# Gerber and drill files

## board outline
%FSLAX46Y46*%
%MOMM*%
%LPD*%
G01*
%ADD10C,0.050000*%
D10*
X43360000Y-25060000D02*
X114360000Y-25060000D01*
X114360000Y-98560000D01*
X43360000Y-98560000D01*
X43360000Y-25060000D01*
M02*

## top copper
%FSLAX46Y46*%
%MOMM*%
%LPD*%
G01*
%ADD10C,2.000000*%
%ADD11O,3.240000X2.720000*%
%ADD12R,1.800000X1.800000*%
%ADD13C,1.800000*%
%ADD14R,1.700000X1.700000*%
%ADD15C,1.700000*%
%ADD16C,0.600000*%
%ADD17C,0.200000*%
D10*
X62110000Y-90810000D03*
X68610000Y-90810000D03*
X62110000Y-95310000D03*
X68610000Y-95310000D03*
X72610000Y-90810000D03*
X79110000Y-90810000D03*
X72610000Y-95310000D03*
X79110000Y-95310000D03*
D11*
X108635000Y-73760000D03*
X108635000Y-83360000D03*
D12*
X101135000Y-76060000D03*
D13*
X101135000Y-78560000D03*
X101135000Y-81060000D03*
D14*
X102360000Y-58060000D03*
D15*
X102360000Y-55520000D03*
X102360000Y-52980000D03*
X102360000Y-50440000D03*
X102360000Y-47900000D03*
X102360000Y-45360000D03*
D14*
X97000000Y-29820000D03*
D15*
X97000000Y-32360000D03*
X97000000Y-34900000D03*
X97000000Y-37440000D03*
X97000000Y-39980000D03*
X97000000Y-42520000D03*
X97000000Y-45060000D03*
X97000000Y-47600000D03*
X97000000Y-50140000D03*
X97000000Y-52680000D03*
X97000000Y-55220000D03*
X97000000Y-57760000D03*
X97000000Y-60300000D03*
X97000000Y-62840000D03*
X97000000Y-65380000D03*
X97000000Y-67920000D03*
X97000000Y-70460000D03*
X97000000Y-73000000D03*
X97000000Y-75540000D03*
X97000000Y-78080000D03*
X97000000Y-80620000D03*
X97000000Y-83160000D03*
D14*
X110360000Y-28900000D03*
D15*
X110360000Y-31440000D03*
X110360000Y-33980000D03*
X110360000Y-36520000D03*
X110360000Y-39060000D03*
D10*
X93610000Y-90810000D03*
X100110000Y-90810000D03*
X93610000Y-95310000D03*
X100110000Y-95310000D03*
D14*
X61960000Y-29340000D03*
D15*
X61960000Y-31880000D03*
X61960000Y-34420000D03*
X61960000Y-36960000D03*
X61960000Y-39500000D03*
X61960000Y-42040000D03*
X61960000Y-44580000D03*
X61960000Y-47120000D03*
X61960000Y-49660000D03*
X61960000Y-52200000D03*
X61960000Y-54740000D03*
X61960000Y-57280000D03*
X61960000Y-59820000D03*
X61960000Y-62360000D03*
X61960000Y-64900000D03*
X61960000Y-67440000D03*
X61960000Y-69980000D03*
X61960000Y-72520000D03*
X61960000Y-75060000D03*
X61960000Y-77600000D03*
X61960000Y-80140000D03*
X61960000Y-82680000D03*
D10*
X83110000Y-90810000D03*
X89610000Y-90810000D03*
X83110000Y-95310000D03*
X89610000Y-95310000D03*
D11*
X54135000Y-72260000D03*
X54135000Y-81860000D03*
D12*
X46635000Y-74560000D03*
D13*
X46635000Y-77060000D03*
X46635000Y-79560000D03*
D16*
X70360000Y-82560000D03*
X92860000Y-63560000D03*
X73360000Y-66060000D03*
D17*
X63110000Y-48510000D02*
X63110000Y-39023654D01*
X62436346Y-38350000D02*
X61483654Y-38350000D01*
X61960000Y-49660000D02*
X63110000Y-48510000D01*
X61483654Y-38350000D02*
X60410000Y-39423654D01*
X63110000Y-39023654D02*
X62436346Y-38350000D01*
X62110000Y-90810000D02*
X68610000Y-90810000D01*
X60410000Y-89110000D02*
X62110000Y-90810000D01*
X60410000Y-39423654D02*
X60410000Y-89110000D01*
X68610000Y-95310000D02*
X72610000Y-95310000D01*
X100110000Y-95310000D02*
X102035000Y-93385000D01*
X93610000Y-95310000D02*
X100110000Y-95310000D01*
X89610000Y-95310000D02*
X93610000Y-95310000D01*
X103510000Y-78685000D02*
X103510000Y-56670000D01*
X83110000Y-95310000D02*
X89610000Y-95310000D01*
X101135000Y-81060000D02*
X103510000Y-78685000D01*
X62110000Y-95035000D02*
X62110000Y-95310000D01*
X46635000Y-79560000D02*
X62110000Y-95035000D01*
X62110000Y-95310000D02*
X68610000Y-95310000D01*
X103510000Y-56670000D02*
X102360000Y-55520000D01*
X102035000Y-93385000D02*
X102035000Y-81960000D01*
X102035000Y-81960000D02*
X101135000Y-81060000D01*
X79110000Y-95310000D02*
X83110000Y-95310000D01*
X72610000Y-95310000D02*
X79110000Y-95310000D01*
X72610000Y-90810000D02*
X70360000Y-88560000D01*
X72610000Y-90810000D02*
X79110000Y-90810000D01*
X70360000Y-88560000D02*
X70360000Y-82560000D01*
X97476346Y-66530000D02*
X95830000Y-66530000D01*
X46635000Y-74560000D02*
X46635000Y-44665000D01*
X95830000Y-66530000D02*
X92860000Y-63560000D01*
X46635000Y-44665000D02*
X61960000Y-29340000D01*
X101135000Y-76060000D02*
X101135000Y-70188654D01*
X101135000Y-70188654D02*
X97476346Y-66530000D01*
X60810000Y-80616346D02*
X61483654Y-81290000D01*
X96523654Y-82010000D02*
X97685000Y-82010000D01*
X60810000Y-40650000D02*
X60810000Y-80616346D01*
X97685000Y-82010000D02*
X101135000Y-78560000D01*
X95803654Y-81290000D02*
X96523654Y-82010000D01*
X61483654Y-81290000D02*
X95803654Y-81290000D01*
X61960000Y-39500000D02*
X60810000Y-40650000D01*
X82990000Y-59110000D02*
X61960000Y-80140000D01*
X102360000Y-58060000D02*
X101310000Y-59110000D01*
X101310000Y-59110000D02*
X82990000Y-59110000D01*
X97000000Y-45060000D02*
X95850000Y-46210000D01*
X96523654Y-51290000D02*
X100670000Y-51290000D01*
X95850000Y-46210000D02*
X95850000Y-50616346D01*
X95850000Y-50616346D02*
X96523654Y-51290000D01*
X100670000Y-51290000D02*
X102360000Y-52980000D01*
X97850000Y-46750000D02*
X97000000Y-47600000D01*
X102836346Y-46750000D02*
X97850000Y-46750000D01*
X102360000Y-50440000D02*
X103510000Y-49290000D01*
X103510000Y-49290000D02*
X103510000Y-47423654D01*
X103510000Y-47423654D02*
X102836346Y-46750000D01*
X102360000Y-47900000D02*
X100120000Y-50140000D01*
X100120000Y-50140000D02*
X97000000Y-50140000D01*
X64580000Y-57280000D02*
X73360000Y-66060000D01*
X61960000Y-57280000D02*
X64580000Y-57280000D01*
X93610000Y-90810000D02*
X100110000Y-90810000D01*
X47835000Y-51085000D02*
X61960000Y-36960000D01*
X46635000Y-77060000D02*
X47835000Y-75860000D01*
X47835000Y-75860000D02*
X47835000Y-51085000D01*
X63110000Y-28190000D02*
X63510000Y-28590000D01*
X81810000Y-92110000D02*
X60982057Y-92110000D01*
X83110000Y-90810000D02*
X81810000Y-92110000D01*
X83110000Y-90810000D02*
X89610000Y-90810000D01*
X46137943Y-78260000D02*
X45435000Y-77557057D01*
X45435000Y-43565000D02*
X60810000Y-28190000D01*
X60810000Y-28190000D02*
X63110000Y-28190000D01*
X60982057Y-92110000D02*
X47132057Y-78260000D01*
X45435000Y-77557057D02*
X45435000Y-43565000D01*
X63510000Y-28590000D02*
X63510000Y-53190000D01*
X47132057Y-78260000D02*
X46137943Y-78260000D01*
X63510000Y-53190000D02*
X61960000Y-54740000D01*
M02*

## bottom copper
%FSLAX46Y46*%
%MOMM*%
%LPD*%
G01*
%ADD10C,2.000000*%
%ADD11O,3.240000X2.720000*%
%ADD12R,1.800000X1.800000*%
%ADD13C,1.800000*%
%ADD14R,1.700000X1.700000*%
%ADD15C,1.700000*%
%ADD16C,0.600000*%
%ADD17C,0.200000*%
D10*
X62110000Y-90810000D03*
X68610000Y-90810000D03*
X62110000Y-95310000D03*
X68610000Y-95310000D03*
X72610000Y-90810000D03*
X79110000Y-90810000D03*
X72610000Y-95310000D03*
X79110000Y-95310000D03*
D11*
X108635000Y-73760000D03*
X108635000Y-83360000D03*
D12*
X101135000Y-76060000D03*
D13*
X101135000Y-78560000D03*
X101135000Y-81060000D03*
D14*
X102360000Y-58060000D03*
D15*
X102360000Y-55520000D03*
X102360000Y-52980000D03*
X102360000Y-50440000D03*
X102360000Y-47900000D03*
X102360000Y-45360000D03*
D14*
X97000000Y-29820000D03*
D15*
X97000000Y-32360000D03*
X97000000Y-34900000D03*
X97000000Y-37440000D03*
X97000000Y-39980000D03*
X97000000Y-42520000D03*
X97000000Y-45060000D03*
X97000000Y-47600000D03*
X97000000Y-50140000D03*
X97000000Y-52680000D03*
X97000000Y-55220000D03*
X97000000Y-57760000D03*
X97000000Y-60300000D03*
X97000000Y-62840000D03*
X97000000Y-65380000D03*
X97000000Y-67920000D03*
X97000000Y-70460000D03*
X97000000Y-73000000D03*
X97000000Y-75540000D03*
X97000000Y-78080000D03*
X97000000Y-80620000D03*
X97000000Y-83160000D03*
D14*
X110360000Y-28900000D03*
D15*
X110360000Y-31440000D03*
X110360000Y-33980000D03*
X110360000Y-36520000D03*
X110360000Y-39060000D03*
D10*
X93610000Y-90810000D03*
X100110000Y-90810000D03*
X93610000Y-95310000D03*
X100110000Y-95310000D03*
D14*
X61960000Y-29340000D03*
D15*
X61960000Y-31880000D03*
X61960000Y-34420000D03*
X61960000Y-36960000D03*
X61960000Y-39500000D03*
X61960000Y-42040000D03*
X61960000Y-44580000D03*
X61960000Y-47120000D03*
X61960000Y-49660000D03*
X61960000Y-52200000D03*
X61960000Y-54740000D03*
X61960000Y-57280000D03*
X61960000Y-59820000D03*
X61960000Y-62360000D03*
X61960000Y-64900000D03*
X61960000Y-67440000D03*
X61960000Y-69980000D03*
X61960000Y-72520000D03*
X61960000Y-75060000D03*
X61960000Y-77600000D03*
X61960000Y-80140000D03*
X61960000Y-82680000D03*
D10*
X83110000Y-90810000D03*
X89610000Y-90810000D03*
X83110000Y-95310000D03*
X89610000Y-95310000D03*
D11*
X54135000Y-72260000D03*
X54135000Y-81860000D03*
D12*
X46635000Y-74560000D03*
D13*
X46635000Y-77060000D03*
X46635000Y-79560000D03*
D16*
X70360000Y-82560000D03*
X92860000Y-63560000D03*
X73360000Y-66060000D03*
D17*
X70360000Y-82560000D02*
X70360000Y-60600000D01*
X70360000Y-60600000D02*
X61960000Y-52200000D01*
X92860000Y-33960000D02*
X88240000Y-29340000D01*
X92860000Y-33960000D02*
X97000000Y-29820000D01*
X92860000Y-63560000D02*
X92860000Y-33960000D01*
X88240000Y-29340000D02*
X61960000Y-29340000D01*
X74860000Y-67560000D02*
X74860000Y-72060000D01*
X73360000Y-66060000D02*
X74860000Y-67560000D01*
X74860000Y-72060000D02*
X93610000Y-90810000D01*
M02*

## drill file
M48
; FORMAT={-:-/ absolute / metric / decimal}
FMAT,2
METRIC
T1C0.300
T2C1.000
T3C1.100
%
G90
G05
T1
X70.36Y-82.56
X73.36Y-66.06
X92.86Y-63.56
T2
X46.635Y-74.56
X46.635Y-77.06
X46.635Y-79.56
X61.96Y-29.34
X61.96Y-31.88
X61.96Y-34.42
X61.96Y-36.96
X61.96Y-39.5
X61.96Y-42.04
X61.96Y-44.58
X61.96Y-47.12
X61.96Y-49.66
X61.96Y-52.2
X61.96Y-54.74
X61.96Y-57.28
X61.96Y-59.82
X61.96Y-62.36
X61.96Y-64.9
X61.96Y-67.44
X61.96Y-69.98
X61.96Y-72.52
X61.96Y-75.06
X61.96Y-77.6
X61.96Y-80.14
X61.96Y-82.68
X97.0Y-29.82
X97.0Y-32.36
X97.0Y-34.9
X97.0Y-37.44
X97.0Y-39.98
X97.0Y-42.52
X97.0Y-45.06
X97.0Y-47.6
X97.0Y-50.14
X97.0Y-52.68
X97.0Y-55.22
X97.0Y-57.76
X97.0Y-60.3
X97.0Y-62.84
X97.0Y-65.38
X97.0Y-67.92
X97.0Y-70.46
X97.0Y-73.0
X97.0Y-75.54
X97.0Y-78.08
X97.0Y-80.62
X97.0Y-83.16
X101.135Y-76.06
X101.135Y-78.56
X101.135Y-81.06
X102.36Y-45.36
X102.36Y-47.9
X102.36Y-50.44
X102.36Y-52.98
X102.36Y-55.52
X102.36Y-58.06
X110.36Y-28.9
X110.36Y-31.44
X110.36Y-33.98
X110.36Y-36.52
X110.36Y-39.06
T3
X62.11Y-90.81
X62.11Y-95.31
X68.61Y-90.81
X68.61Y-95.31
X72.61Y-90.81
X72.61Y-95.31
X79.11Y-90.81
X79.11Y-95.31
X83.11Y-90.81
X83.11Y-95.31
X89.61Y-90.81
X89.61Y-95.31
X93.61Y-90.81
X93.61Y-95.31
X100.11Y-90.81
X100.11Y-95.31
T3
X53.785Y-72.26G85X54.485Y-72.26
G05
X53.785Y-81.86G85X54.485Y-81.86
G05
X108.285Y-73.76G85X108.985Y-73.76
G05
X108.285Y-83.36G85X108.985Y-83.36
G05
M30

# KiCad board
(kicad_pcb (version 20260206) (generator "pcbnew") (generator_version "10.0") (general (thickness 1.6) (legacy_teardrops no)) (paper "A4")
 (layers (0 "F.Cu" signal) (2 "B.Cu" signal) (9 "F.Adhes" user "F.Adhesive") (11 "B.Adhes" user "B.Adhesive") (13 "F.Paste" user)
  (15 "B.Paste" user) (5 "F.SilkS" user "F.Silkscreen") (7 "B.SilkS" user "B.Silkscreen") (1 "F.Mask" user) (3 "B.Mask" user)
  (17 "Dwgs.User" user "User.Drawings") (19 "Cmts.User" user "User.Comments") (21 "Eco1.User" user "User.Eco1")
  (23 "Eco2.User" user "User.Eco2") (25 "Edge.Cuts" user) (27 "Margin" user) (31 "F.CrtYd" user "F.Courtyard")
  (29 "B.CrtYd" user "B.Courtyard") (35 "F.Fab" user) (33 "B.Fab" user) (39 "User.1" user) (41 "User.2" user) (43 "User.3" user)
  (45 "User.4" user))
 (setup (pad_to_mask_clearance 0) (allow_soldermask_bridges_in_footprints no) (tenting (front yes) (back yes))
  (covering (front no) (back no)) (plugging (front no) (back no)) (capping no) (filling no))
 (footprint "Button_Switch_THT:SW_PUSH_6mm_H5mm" (layer "F.Cu") (at 62.11 90.81)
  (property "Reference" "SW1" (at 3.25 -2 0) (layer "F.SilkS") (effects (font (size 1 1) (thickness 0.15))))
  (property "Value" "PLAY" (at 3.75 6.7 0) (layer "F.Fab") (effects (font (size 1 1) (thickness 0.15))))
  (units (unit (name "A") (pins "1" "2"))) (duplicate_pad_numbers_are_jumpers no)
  (pad "1" thru_hole circle (at 0 0 90) (size 2 2) (drill 1.1) (layers "*.Cu" "*.Mask") (remove_unused_layers no) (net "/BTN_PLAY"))
  (pad "1" thru_hole circle (at 6.5 0 90) (size 2 2) (drill 1.1) (layers "*.Cu" "*.Mask") (remove_unused_layers no) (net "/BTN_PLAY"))
  (pad "2" thru_hole circle (at 0 4.5 90) (size 2 2) (drill 1.1) (layers "*.Cu" "*.Mask") (remove_unused_layers no) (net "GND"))
  (pad "2" thru_hole circle (at 6.5 4.5 90) (size 2 2) (drill 1.1) (layers "*.Cu" "*.Mask") (remove_unused_layers no) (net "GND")))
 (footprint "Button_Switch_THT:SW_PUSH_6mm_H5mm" (layer "F.Cu") (at 72.61 90.81)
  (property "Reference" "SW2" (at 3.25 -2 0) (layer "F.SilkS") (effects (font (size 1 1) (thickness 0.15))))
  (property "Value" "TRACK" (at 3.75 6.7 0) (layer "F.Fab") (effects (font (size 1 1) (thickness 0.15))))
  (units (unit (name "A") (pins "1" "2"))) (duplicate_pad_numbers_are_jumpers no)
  (pad "1" thru_hole circle (at 0 0 90) (size 2 2) (drill 1.1) (layers "*.Cu" "*.Mask") (remove_unused_layers no) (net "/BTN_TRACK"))
  (pad "1" thru_hole circle (at 6.5 0 90) (size 2 2) (drill 1.1) (layers "*.Cu" "*.Mask") (remove_unused_layers no) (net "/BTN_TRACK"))
  (pad "2" thru_hole circle (at 0 4.5 90) (size 2 2) (drill 1.1) (layers "*.Cu" "*.Mask") (remove_unused_layers no) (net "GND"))
  (pad "2" thru_hole circle (at 6.5 4.5 90) (size 2 2) (drill 1.1) (layers "*.Cu" "*.Mask") (remove_unused_layers no) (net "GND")))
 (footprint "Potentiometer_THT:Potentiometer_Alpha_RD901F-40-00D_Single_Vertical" (layer "F.Cu") (at 101.135 76.06)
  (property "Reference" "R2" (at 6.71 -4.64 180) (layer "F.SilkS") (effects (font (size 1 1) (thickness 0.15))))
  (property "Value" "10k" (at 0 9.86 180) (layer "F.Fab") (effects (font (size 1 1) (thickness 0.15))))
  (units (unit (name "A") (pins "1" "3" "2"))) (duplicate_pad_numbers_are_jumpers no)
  (pad "" thru_hole oval (at 7.5 -2.3 90) (size 2.72 3.24) (drill oval 1.1 1.8) (layers "*.Cu" "*.Mask") (remove_unused_layers no))
  (pad "" thru_hole oval (at 7.5 7.3 90) (size 2.72 3.24) (drill oval 1.1 1.8) (layers "*.Cu" "*.Mask") (remove_unused_layers no))
  (pad "1" thru_hole rect (at 0 0 90) (size 1.8 1.8) (drill 1) (layers "*.Cu" "*.Mask") (remove_unused_layers no) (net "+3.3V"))
  (pad "2" thru_hole circle (at 0 2.5 90) (size 1.8 1.8) (drill 1) (layers "*.Cu" "*.Mask") (remove_unused_layers no) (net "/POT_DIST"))
  (pad "3" thru_hole circle (at 0 5 90) (size 1.8 1.8) (drill 1) (layers "*.Cu" "*.Mask") (remove_unused_layers no) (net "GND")))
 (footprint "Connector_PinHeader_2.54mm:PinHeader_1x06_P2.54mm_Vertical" (layer "F.Cu") (at 102.36 58.06 180)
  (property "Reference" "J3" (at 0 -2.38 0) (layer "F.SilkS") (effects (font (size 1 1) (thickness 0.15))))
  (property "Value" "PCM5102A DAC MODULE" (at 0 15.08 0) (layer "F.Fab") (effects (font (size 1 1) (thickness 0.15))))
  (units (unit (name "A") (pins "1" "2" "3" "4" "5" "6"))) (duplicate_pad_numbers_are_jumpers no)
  (pad "1" thru_hole rect (at 0 0 180) (size 1.7 1.7) (drill 1) (layers "*.Cu" "*.Mask") (remove_unused_layers no) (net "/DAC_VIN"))
  (pad "2" thru_hole circle (at 0 2.54 180) (size 1.7 1.7) (drill 1) (layers "*.Cu" "*.Mask") (remove_unused_layers no) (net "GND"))
  (pad "3" thru_hole circle (at 0 5.08 180) (size 1.7 1.7) (drill 1) (layers "*.Cu" "*.Mask") (remove_unused_layers no) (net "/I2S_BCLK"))
  (pad "4" thru_hole circle (at 0 7.62 180) (size 1.7 1.7) (drill 1) (layers "*.Cu" "*.Mask") (remove_unused_layers no) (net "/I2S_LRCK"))
  (pad "5" thru_hole circle (at 0 10.16 180) (size 1.7 1.7) (drill 1) (layers "*.Cu" "*.Mask") (remove_unused_layers no) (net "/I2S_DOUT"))
  (pad "6" thru_hole circle (at 0 12.7 180) (size 1.7 1.7) (drill 1) (layers "*.Cu" "*.Mask") (remove_unused_layers no) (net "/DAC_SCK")))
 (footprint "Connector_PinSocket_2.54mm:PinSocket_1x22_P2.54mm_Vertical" (layer "F.Cu") (at 97 29.82)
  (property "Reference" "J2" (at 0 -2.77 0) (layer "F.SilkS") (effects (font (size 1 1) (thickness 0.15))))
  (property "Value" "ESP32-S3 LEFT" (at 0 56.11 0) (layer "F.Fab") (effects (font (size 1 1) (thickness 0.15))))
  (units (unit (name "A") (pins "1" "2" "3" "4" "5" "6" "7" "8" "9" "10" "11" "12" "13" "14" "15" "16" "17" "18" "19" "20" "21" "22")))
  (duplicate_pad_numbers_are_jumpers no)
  (pad "1" thru_hole rect (at 0 0) (size 1.7 1.7) (drill 1) (layers "*.Cu" "*.Mask") (remove_unused_layers no) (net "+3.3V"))
  (pad "2" thru_hole circle (at 0 2.54) (size 1.7 1.7) (drill 1) (layers "*.Cu" "*.Mask") (remove_unused_layers no)
   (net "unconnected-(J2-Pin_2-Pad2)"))
  (pad "3" thru_hole circle (at 0 5.08) (size 1.7 1.7) (drill 1) (layers "*.Cu" "*.Mask") (remove_unused_layers no)
   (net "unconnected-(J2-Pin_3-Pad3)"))
  (pad "4" thru_hole circle (at 0 7.62) (size 1.7 1.7) (drill 1) (layers "*.Cu" "*.Mask") (remove_unused_layers no)
   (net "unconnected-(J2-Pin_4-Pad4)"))
  (pad "5" thru_hole circle (at 0 10.16) (size 1.7 1.7) (drill 1) (layers "*.Cu" "*.Mask") (remove_unused_layers no)
   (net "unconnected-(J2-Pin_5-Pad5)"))
  (pad "6" thru_hole circle (at 0 12.7) (size 1.7 1.7) (drill 1) (layers "*.Cu" "*.Mask") (remove_unused_layers no)
   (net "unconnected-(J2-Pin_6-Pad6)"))
  (pad "7" thru_hole circle (at 0 15.24) (size 1.7 1.7) (drill 1) (layers "*.Cu" "*.Mask") (remove_unused_layers no) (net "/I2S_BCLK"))
  (pad "8" thru_hole circle (at 0 17.78) (size 1.7 1.7) (drill 1) (layers "*.Cu" "*.Mask") (remove_unused_layers no) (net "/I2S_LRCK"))
  (pad "9" thru_hole circle (at 0 20.32) (size 1.7 1.7) (drill 1) (layers "*.Cu" "*.Mask") (remove_unused_layers no) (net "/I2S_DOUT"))
  (pad "10" thru_hole circle (at 0 22.86) (size 1.7 1.7) (drill 1) (layers "*.Cu" "*.Mask") (remove_unused_layers no)
   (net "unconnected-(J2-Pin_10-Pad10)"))
  (pad "11" thru_hole circle (at 0 25.4) (size 1.7 1.7) (drill 1) (layers "*.Cu" "*.Mask") (remove_unused_layers no)
   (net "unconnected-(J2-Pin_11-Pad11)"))
  (pad "12" thru_hole circle (at 0 27.94) (size 1.7 1.7) (drill 1) (layers "*.Cu" "*.Mask") (remove_unused_layers no)
   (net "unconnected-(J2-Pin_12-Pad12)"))
  (pad "13" thru_hole circle (at 0 30.48) (size 1.7 1.7) (drill 1) (layers "*.Cu" "*.Mask") (remove_unused_layers no)
   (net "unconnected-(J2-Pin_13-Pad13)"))
  (pad "14" thru_hole circle (at 0 33.02) (size 1.7 1.7) (drill 1) (layers "*.Cu" "*.Mask") (remove_unused_layers no)
   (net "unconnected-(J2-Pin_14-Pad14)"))
  (pad "15" thru_hole circle (at 0 35.56) (size 1.7 1.7) (drill 1) (layers "*.Cu" "*.Mask") (remove_unused_layers no)
   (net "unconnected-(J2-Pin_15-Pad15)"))
  (pad "16" thru_hole circle (at 0 38.1) (size 1.7 1.7) (drill 1) (layers "*.Cu" "*.Mask") (remove_unused_layers no)
   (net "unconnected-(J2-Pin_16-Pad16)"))
  (pad "17" thru_hole circle (at 0 40.64) (size 1.7 1.7) (drill 1) (layers "*.Cu" "*.Mask") (remove_unused_layers no)
   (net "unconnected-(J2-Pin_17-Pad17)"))
  (pad "18" thru_hole circle (at 0 43.18) (size 1.7 1.7) (drill 1) (layers "*.Cu" "*.Mask") (remove_unused_layers no)
   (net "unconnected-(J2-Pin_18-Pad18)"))
  (pad "19" thru_hole circle (at 0 45.72) (size 1.7 1.7) (drill 1) (layers "*.Cu" "*.Mask") (remove_unused_layers no)
   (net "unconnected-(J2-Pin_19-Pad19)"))
  (pad "20" thru_hole circle (at 0 48.26) (size 1.7 1.7) (drill 1) (layers "*.Cu" "*.Mask") (remove_unused_layers no)
   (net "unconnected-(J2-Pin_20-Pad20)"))
  (pad "21" thru_hole circle (at 0 50.8) (size 1.7 1.7) (drill 1) (layers "*.Cu" "*.Mask") (remove_unused_layers no)
   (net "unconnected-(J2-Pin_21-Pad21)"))
  (pad "22" thru_hole circle (at 0 53.34) (size 1.7 1.7) (drill 1) (layers "*.Cu" "*.Mask") (remove_unused_layers no)
   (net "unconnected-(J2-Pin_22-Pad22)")))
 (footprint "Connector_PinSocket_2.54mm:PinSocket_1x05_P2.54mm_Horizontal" (layer "F.Cu") (at 110.36 28.9)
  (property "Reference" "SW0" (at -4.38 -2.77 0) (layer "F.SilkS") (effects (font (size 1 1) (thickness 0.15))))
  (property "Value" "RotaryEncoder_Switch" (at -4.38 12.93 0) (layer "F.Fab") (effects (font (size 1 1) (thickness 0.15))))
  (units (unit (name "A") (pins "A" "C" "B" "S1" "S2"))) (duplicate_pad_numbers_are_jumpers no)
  (pad "1" thru_hole rect (at 0 0) (size 1.7 1.7) (drill 1) (layers "*.Cu" "*.Mask") (remove_unused_layers no))
  (pad "2" thru_hole circle (at 0 2.54) (size 1.7 1.7) (drill 1) (layers "*.Cu" "*.Mask") (remove_unused_layers no))
  (pad "3" thru_hole circle (at 0 5.08) (size 1.7 1.7) (drill 1) (layers "*.Cu" "*.Mask") (remove_unused_layers no))
  (pad "4" thru_hole circle (at 0 7.62) (size 1.7 1.7) (drill 1) (layers "*.Cu" "*.Mask") (remove_unused_layers no))
  (pad "5" thru_hole circle (at 0 10.16) (size 1.7 1.7) (drill 1) (layers "*.Cu" "*.Mask") (remove_unused_layers no)))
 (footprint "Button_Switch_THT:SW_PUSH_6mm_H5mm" (layer "F.Cu") (at 93.61 90.81)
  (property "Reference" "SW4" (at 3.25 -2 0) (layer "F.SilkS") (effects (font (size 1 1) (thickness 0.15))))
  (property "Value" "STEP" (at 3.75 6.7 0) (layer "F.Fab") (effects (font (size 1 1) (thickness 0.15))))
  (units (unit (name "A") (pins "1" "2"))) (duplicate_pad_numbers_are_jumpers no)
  (pad "1" thru_hole circle (at 0 0 90) (size 2 2) (drill 1.1) (layers "*.Cu" "*.Mask") (remove_unused_layers no) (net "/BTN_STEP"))
  (pad "1" thru_hole circle (at 6.5 0 90) (size 2 2) (drill 1.1) (layers "*.Cu" "*.Mask") (remove_unused_layers no) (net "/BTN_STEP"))
  (pad "2" thru_hole circle (at 0 4.5 90) (size 2 2) (drill 1.1) (layers "*.Cu" "*.Mask") (remove_unused_layers no) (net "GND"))
  (pad "2" thru_hole circle (at 6.5 4.5 90) (size 2 2) (drill 1.1) (layers "*.Cu" "*.Mask") (remove_unused_layers no) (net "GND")))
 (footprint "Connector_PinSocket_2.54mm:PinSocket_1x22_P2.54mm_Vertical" (layer "F.Cu") (at 61.96 29.34)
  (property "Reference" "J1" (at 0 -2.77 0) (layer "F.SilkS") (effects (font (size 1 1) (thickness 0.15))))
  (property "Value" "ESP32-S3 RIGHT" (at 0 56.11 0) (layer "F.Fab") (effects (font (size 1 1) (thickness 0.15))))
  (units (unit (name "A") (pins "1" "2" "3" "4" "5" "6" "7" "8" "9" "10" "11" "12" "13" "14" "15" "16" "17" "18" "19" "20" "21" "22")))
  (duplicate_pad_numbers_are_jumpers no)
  (pad "1" thru_hole rect (at 0 0) (size 1.7 1.7) (drill 1) (layers "*.Cu" "*.Mask") (remove_unused_layers no) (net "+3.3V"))
  (pad "2" thru_hole circle (at 0 2.54) (size 1.7 1.7) (drill 1) (layers "*.Cu" "*.Mask") (remove_unused_layers no)
   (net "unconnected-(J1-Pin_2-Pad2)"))
  (pad "3" thru_hole circle (at 0 5.08) (size 1.7 1.7) (drill 1) (layers "*.Cu" "*.Mask") (remove_unused_layers no)
   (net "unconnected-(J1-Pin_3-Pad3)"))
  (pad "4" thru_hole circle (at 0 7.62) (size 1.7 1.7) (drill 1) (layers "*.Cu" "*.Mask") (remove_unused_layers no) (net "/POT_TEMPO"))
  (pad "5" thru_hole circle (at 0 10.16) (size 1.7 1.7) (drill 1) (layers "*.Cu" "*.Mask") (remove_unused_layers no) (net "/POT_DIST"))
  (pad "6" thru_hole circle (at 0 12.7) (size 1.7 1.7) (drill 1) (layers "*.Cu" "*.Mask") (remove_unused_layers no) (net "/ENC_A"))
  (pad "7" thru_hole circle (at 0 15.24) (size 1.7 1.7) (drill 1) (layers "*.Cu" "*.Mask") (remove_unused_layers no) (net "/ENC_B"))
  (pad "8" thru_hole circle (at 0 17.78) (size 1.7 1.7) (drill 1) (layers "*.Cu" "*.Mask") (remove_unused_layers no) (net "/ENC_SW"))
  (pad "9" thru_hole circle (at 0 20.32) (size 1.7 1.7) (drill 1) (layers "*.Cu" "*.Mask") (remove_unused_layers no) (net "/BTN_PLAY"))
  (pad "10" thru_hole circle (at 0 22.86) (size 1.7 1.7) (drill 1) (layers "*.Cu" "*.Mask") (remove_unused_layers no) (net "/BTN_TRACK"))
  (pad "11" thru_hole circle (at 0 25.4) (size 1.7 1.7) (drill 1) (layers "*.Cu" "*.Mask") (remove_unused_layers no) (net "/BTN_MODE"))
  (pad "12" thru_hole circle (at 0 27.94) (size 1.7 1.7) (drill 1) (layers "*.Cu" "*.Mask") (remove_unused_layers no) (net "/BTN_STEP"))
  (pad "13" thru_hole circle (at 0 30.48) (size 1.7 1.7) (drill 1) (layers "*.Cu" "*.Mask") (remove_unused_layers no)
   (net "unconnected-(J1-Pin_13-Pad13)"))
  (pad "14" thru_hole circle (at 0 33.02) (size 1.7 1.7) (drill 1) (layers "*.Cu" "*.Mask") (remove_unused_layers no)
   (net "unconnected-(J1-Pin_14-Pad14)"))
  (pad "15" thru_hole circle (at 0 35.56) (size 1.7 1.7) (drill 1) (layers "*.Cu" "*.Mask") (remove_unused_layers no)
   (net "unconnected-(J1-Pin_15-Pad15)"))
  (pad "16" thru_hole circle (at 0 38.1) (size 1.7 1.7) (drill 1) (layers "*.Cu" "*.Mask") (remove_unused_layers no)
   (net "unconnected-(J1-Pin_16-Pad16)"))
  (pad "17" thru_hole circle (at 0 40.64) (size 1.7 1.7) (drill 1) (layers "*.Cu" "*.Mask") (remove_unused_layers no)
   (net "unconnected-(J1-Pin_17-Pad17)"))
  (pad "18" thru_hole circle (at 0 43.18) (size 1.7 1.7) (drill 1) (layers "*.Cu" "*.Mask") (remove_unused_layers no)
   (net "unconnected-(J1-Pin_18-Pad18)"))
  (pad "19" thru_hole circle (at 0 45.72) (size 1.7 1.7) (drill 1) (layers "*.Cu" "*.Mask") (remove_unused_layers no)
   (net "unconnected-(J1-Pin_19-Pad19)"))
  (pad "20" thru_hole circle (at 0 48.26) (size 1.7 1.7) (drill 1) (layers "*.Cu" "*.Mask") (remove_unused_layers no)
   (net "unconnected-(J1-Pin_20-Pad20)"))
  (pad "21" thru_hole circle (at 0 50.8) (size 1.7 1.7) (drill 1) (layers "*.Cu" "*.Mask") (remove_unused_layers no) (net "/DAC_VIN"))
  (pad "22" thru_hole circle (at 0 53.34) (size 1.7 1.7) (drill 1) (layers "*.Cu" "*.Mask") (remove_unused_layers no)
   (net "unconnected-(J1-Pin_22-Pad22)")))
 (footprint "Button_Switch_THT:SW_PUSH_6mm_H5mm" (layer "F.Cu") (at 83.11 90.81)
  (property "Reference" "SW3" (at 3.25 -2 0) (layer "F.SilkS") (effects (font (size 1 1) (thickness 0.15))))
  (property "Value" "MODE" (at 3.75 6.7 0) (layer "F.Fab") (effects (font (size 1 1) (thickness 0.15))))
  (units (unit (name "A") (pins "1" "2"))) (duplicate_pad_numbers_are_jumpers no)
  (pad "1" thru_hole circle (at 0 0 90) (size 2 2) (drill 1.1) (layers "*.Cu" "*.Mask") (remove_unused_layers no) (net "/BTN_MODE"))
  (pad "1" thru_hole circle (at 6.5 0 90) (size 2 2) (drill 1.1) (layers "*.Cu" "*.Mask") (remove_unused_layers no) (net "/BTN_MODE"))
  (pad "2" thru_hole circle (at 0 4.5 90) (size 2 2) (drill 1.1) (layers "*.Cu" "*.Mask") (remove_unused_layers no) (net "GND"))
  (pad "2" thru_hole circle (at 6.5 4.5 90) (size 2 2) (drill 1.1) (layers "*.Cu" "*.Mask") (remove_unused_layers no) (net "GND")))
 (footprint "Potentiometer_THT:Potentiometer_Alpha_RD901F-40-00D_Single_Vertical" (layer "F.Cu") (at 46.635 74.56)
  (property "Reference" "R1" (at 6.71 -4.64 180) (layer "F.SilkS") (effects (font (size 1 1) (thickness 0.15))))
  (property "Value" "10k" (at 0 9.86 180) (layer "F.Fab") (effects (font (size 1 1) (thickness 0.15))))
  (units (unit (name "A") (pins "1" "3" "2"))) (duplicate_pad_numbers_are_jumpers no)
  (pad "" thru_hole oval (at 7.5 -2.3 90) (size 2.72 3.24) (drill oval 1.1 1.8) (layers "*.Cu" "*.Mask") (remove_unused_layers no))
  (pad "" thru_hole oval (at 7.5 7.3 90) (size 2.72 3.24) (drill oval 1.1 1.8) (layers "*.Cu" "*.Mask") (remove_unused_layers no))
  (pad "1" thru_hole rect (at 0 0 90) (size 1.8 1.8) (drill 1) (layers "*.Cu" "*.Mask") (remove_unused_layers no) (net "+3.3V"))
  (pad "2" thru_hole circle (at 0 2.5 90) (size 1.8 1.8) (drill 1) (layers "*.Cu" "*.Mask") (remove_unused_layers no) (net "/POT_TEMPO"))
  (pad "3" thru_hole circle (at 0 5 90) (size 1.8 1.8) (drill 1) (layers "*.Cu" "*.Mask") (remove_unused_layers no) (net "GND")))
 (gr_rect (start 43.36 25.06) (end 114.36 98.56) (stroke (width 0.05) (type default)) (fill no) (layer "Edge.Cuts"))
 (segment (start 63.11 48.51) (end 63.11 39.023654) (width 0.2) (layer "F.Cu") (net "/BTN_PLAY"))
 (segment (start 62.436346 38.35) (end 61.483654 38.35) (width 0.2) (layer "F.Cu") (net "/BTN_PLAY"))
 (segment (start 61.96 49.66) (end 63.11 48.51) (width 0.2) (layer "F.Cu") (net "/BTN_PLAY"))
 (segment (start 61.483654 38.35) (end 60.41 39.423654) (width 0.2) (layer "F.Cu") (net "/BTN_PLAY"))
 (segment (start 63.11 39.023654) (end 62.436346 38.35) (width 0.2) (layer "F.Cu") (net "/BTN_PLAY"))
 (segment (start 62.11 90.81) (end 68.61 90.81) (width 0.2) (layer "F.Cu") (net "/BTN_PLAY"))
 (segment (start 60.41 89.11) (end 62.11 90.81) (width 0.2) (layer "F.Cu") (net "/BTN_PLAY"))
 (segment (start 60.41 39.423654) (end 60.41 89.11) (width 0.2) (layer "F.Cu") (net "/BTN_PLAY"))
 (segment (start 68.61 95.31) (end 72.61 95.31) (width 0.2) (layer "F.Cu") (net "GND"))
 (segment (start 100.11 95.31) (end 102.035 93.385) (width 0.2) (layer "F.Cu") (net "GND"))
 (segment (start 93.61 95.31) (end 100.11 95.31) (width 0.2) (layer "F.Cu") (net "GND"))
 (segment (start 89.61 95.31) (end 93.61 95.31) (width 0.2) (layer "F.Cu") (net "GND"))
 (segment (start 103.51 78.685) (end 103.51 56.67) (width 0.2) (layer "F.Cu") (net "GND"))
 (segment (start 83.11 95.31) (end 89.61 95.31) (width 0.2) (layer "F.Cu") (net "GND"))
 (segment (start 101.135 81.06) (end 103.51 78.685) (width 0.2) (layer "F.Cu") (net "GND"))
 (segment (start 62.11 95.035) (end 62.11 95.31) (width 0.2) (layer "F.Cu") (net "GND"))
 (segment (start 46.635 79.56) (end 62.11 95.035) (width 0.2) (layer "F.Cu") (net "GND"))
 (segment (start 62.11 95.31) (end 68.61 95.31) (width 0.2) (layer "F.Cu") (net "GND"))
 (segment (start 103.51 56.67) (end 102.36 55.52) (width 0.2) (layer "F.Cu") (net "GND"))
 (segment (start 102.035 93.385) (end 102.035 81.96) (width 0.2) (layer "F.Cu") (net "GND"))
 (segment (start 102.035 81.96) (end 101.135 81.06) (width 0.2) (layer "F.Cu") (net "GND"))
 (segment (start 79.11 95.31) (end 83.11 95.31) (width 0.2) (layer "F.Cu") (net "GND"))
 (segment (start 72.61 95.31) (end 79.11 95.31) (width 0.2) (layer "F.Cu") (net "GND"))
 (segment (start 72.61 90.81) (end 70.36 88.56) (width 0.2) (layer "F.Cu") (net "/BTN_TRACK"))
 (segment (start 72.61 90.81) (end 79.11 90.81) (width 0.2) (layer "F.Cu") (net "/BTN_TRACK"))
 (segment (start 70.36 88.56) (end 70.36 82.56) (width 0.2) (layer "F.Cu") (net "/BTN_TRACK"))
 (via (at 70.36 82.56) (size 0.6) (drill 0.3) (layers "F.Cu" "B.Cu") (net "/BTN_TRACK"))
 (segment (start 70.36 82.56) (end 70.36 60.6) (width 0.2) (layer "B.Cu") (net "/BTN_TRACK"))
 (segment (start 70.36 60.6) (end 61.96 52.2) (width 0.2) (layer "B.Cu") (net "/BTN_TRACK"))
 (segment (start 97.476346 66.53) (end 95.83 66.53) (width 0.2) (layer "F.Cu") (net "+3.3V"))
 (segment (start 46.635 74.56) (end 46.635 44.665) (width 0.2) (layer "F.Cu") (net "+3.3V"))
 (segment (start 95.83 66.53) (end 92.86 63.56) (width 0.2) (layer "F.Cu") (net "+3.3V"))
 (segment (start 46.635 44.665) (end 61.96 29.34) (width 0.2) (layer "F.Cu") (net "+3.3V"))
 (segment (start 101.135 76.06) (end 101.135 70.188654) (width 0.2) (layer "F.Cu") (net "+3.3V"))
 (segment (start 101.135 70.188654) (end 97.476346 66.53) (width 0.2) (layer "F.Cu") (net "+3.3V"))
 (via (at 92.86 63.56) (size 0.6) (drill 0.3) (layers "F.Cu" "B.Cu") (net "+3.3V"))
 (segment (start 92.86 33.96) (end 88.24 29.34) (width 0.2) (layer "B.Cu") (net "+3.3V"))
 (segment (start 92.86 33.96) (end 97 29.82) (width 0.2) (layer "B.Cu") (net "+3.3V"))
 (segment (start 92.86 63.56) (end 92.86 33.96) (width 0.2) (layer "B.Cu") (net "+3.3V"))
 (segment (start 88.24 29.34) (end 61.96 29.34) (width 0.2) (layer "B.Cu") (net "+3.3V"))
 (segment (start 60.81 80.616346) (end 61.483654 81.29) (width 0.2) (layer "F.Cu") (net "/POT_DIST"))
 (segment (start 96.523654 82.01) (end 97.685 82.01) (width 0.2) (layer "F.Cu") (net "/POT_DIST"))
 (segment (start 60.81 40.65) (end 60.81 80.616346) (width 0.2) (layer "F.Cu") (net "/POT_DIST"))
 (segment (start 97.685 82.01) (end 101.135 78.56) (width 0.2) (layer "F.Cu") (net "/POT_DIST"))
 (segment (start 95.803654 81.29) (end 96.523654 82.01) (width 0.2) (layer "F.Cu") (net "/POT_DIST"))
 (segment (start 61.483654 81.29) (end 95.803654 81.29) (width 0.2) (layer "F.Cu") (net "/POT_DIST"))
 (segment (start 61.96 39.5) (end 60.81 40.65) (width 0.2) (layer "F.Cu") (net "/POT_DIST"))
 (segment (start 82.99 59.11) (end 61.96 80.14) (width 0.2) (layer "F.Cu") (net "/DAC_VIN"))
 (segment (start 102.36 58.06) (end 101.31 59.11) (width 0.2) (layer "F.Cu") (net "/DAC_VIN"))
 (segment (start 101.31 59.11) (end 82.99 59.11) (width 0.2) (layer "F.Cu") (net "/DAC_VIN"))
 (segment (start 97 45.06) (end 95.85 46.21) (width 0.2) (layer "F.Cu") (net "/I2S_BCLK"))
 (segment (start 96.523654 51.29) (end 100.67 51.29) (width 0.2) (layer "F.Cu") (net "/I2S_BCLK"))
 (segment (start 95.85 46.21) (end 95.85 50.616346) (width 0.2) (layer "F.Cu") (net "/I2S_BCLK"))
 (segment (start 95.85 50.616346) (end 96.523654 51.29) (width 0.2) (layer "F.Cu") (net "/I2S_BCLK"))
 (segment (start 100.67 51.29) (end 102.36 52.98) (width 0.2) (layer "F.Cu") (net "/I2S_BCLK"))
 (segment (start 97.85 46.75) (end 97 47.6) (width 0.2) (layer "F.Cu") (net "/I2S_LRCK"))
 (segment (start 102.836346 46.75) (end 97.85 46.75) (width 0.2) (layer "F.Cu") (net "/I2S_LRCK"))
 (segment (start 102.36 50.44) (end 103.51 49.29) (width 0.2) (layer "F.Cu") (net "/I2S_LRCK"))
 (segment (start 103.51 49.29) (end 103.51 47.423654) (width 0.2) (layer "F.Cu") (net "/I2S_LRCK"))
 (segment (start 103.51 47.423654) (end 102.836346 46.75) (width 0.2) (layer "F.Cu") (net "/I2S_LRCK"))
 (segment (start 102.36 47.9) (end 100.12 50.14) (width 0.2) (layer "F.Cu") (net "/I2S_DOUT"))
 (segment (start 100.12 50.14) (end 97 50.14) (width 0.2) (layer "F.Cu") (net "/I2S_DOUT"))
 (segment (start 64.58 57.28) (end 73.36 66.06) (width 0.2) (layer "F.Cu") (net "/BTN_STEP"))
 (segment (start 61.96 57.28) (end 64.58 57.28) (width 0.2) (layer "F.Cu") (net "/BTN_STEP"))
 (segment (start 93.61 90.81) (end 100.11 90.81) (width 0.2) (layer "F.Cu") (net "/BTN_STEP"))
 (via (at 73.36 66.06) (size 0.6) (drill 0.3) (layers "F.Cu" "B.Cu") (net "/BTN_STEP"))
 (segment (start 74.86 67.56) (end 74.86 72.06) (width 0.2) (layer "B.Cu") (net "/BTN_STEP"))
 (segment (start 73.36 66.06) (end 74.86 67.56) (width 0.2) (layer "B.Cu") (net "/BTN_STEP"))
 (segment (start 74.86 72.06) (end 93.61 90.81) (width 0.2) (layer "B.Cu") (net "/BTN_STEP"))
 (segment (start 47.835 51.085) (end 61.96 36.96) (width 0.2) (layer "F.Cu") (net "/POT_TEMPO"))
 (segment (start 46.635 77.06) (end 47.835 75.86) (width 0.2) (layer "F.Cu") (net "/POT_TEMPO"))
 (segment (start 47.835 75.86) (end 47.835 51.085) (width 0.2) (layer "F.Cu") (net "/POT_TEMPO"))
 (segment (start 63.11 28.19) (end 63.51 28.59) (width 0.2) (layer "F.Cu") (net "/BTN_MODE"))
 (segment (start 81.81 92.11) (end 60.982057 92.11) (width 0.2) (layer "F.Cu") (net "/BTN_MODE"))
 (segment (start 83.11 90.81) (end 81.81 92.11) (width 0.2) (layer "F.Cu") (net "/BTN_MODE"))
 (segment (start 83.11 90.81) (end 89.61 90.81) (width 0.2) (layer "F.Cu") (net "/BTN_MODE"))
 (segment (start 46.137943 78.26) (end 45.435 77.557057) (width 0.2) (layer "F.Cu") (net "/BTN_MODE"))
 (segment (start 45.435 43.565) (end 60.81 28.19) (width 0.2) (layer "F.Cu") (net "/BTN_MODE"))
 (segment (start 60.81 28.19) (end 63.11 28.19) (width 0.2) (layer "F.Cu") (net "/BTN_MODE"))
 (segment (start 60.982057 92.11) (end 47.132057 78.26) (width 0.2) (layer "F.Cu") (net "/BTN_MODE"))
 (segment (start 45.435 77.557057) (end 45.435 43.565) (width 0.2) (layer "F.Cu") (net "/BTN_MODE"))
 (segment (start 63.51 28.59) (end 63.51 53.19) (width 0.2) (layer "F.Cu") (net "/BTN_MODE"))
 (segment (start 47.132057 78.26) (end 46.137943 78.26) (width 0.2) (layer "F.Cu") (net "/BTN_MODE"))
 (segment (start 63.51 53.19) (end 61.96 54.74) (width 0.2) (layer "F.Cu") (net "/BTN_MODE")))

